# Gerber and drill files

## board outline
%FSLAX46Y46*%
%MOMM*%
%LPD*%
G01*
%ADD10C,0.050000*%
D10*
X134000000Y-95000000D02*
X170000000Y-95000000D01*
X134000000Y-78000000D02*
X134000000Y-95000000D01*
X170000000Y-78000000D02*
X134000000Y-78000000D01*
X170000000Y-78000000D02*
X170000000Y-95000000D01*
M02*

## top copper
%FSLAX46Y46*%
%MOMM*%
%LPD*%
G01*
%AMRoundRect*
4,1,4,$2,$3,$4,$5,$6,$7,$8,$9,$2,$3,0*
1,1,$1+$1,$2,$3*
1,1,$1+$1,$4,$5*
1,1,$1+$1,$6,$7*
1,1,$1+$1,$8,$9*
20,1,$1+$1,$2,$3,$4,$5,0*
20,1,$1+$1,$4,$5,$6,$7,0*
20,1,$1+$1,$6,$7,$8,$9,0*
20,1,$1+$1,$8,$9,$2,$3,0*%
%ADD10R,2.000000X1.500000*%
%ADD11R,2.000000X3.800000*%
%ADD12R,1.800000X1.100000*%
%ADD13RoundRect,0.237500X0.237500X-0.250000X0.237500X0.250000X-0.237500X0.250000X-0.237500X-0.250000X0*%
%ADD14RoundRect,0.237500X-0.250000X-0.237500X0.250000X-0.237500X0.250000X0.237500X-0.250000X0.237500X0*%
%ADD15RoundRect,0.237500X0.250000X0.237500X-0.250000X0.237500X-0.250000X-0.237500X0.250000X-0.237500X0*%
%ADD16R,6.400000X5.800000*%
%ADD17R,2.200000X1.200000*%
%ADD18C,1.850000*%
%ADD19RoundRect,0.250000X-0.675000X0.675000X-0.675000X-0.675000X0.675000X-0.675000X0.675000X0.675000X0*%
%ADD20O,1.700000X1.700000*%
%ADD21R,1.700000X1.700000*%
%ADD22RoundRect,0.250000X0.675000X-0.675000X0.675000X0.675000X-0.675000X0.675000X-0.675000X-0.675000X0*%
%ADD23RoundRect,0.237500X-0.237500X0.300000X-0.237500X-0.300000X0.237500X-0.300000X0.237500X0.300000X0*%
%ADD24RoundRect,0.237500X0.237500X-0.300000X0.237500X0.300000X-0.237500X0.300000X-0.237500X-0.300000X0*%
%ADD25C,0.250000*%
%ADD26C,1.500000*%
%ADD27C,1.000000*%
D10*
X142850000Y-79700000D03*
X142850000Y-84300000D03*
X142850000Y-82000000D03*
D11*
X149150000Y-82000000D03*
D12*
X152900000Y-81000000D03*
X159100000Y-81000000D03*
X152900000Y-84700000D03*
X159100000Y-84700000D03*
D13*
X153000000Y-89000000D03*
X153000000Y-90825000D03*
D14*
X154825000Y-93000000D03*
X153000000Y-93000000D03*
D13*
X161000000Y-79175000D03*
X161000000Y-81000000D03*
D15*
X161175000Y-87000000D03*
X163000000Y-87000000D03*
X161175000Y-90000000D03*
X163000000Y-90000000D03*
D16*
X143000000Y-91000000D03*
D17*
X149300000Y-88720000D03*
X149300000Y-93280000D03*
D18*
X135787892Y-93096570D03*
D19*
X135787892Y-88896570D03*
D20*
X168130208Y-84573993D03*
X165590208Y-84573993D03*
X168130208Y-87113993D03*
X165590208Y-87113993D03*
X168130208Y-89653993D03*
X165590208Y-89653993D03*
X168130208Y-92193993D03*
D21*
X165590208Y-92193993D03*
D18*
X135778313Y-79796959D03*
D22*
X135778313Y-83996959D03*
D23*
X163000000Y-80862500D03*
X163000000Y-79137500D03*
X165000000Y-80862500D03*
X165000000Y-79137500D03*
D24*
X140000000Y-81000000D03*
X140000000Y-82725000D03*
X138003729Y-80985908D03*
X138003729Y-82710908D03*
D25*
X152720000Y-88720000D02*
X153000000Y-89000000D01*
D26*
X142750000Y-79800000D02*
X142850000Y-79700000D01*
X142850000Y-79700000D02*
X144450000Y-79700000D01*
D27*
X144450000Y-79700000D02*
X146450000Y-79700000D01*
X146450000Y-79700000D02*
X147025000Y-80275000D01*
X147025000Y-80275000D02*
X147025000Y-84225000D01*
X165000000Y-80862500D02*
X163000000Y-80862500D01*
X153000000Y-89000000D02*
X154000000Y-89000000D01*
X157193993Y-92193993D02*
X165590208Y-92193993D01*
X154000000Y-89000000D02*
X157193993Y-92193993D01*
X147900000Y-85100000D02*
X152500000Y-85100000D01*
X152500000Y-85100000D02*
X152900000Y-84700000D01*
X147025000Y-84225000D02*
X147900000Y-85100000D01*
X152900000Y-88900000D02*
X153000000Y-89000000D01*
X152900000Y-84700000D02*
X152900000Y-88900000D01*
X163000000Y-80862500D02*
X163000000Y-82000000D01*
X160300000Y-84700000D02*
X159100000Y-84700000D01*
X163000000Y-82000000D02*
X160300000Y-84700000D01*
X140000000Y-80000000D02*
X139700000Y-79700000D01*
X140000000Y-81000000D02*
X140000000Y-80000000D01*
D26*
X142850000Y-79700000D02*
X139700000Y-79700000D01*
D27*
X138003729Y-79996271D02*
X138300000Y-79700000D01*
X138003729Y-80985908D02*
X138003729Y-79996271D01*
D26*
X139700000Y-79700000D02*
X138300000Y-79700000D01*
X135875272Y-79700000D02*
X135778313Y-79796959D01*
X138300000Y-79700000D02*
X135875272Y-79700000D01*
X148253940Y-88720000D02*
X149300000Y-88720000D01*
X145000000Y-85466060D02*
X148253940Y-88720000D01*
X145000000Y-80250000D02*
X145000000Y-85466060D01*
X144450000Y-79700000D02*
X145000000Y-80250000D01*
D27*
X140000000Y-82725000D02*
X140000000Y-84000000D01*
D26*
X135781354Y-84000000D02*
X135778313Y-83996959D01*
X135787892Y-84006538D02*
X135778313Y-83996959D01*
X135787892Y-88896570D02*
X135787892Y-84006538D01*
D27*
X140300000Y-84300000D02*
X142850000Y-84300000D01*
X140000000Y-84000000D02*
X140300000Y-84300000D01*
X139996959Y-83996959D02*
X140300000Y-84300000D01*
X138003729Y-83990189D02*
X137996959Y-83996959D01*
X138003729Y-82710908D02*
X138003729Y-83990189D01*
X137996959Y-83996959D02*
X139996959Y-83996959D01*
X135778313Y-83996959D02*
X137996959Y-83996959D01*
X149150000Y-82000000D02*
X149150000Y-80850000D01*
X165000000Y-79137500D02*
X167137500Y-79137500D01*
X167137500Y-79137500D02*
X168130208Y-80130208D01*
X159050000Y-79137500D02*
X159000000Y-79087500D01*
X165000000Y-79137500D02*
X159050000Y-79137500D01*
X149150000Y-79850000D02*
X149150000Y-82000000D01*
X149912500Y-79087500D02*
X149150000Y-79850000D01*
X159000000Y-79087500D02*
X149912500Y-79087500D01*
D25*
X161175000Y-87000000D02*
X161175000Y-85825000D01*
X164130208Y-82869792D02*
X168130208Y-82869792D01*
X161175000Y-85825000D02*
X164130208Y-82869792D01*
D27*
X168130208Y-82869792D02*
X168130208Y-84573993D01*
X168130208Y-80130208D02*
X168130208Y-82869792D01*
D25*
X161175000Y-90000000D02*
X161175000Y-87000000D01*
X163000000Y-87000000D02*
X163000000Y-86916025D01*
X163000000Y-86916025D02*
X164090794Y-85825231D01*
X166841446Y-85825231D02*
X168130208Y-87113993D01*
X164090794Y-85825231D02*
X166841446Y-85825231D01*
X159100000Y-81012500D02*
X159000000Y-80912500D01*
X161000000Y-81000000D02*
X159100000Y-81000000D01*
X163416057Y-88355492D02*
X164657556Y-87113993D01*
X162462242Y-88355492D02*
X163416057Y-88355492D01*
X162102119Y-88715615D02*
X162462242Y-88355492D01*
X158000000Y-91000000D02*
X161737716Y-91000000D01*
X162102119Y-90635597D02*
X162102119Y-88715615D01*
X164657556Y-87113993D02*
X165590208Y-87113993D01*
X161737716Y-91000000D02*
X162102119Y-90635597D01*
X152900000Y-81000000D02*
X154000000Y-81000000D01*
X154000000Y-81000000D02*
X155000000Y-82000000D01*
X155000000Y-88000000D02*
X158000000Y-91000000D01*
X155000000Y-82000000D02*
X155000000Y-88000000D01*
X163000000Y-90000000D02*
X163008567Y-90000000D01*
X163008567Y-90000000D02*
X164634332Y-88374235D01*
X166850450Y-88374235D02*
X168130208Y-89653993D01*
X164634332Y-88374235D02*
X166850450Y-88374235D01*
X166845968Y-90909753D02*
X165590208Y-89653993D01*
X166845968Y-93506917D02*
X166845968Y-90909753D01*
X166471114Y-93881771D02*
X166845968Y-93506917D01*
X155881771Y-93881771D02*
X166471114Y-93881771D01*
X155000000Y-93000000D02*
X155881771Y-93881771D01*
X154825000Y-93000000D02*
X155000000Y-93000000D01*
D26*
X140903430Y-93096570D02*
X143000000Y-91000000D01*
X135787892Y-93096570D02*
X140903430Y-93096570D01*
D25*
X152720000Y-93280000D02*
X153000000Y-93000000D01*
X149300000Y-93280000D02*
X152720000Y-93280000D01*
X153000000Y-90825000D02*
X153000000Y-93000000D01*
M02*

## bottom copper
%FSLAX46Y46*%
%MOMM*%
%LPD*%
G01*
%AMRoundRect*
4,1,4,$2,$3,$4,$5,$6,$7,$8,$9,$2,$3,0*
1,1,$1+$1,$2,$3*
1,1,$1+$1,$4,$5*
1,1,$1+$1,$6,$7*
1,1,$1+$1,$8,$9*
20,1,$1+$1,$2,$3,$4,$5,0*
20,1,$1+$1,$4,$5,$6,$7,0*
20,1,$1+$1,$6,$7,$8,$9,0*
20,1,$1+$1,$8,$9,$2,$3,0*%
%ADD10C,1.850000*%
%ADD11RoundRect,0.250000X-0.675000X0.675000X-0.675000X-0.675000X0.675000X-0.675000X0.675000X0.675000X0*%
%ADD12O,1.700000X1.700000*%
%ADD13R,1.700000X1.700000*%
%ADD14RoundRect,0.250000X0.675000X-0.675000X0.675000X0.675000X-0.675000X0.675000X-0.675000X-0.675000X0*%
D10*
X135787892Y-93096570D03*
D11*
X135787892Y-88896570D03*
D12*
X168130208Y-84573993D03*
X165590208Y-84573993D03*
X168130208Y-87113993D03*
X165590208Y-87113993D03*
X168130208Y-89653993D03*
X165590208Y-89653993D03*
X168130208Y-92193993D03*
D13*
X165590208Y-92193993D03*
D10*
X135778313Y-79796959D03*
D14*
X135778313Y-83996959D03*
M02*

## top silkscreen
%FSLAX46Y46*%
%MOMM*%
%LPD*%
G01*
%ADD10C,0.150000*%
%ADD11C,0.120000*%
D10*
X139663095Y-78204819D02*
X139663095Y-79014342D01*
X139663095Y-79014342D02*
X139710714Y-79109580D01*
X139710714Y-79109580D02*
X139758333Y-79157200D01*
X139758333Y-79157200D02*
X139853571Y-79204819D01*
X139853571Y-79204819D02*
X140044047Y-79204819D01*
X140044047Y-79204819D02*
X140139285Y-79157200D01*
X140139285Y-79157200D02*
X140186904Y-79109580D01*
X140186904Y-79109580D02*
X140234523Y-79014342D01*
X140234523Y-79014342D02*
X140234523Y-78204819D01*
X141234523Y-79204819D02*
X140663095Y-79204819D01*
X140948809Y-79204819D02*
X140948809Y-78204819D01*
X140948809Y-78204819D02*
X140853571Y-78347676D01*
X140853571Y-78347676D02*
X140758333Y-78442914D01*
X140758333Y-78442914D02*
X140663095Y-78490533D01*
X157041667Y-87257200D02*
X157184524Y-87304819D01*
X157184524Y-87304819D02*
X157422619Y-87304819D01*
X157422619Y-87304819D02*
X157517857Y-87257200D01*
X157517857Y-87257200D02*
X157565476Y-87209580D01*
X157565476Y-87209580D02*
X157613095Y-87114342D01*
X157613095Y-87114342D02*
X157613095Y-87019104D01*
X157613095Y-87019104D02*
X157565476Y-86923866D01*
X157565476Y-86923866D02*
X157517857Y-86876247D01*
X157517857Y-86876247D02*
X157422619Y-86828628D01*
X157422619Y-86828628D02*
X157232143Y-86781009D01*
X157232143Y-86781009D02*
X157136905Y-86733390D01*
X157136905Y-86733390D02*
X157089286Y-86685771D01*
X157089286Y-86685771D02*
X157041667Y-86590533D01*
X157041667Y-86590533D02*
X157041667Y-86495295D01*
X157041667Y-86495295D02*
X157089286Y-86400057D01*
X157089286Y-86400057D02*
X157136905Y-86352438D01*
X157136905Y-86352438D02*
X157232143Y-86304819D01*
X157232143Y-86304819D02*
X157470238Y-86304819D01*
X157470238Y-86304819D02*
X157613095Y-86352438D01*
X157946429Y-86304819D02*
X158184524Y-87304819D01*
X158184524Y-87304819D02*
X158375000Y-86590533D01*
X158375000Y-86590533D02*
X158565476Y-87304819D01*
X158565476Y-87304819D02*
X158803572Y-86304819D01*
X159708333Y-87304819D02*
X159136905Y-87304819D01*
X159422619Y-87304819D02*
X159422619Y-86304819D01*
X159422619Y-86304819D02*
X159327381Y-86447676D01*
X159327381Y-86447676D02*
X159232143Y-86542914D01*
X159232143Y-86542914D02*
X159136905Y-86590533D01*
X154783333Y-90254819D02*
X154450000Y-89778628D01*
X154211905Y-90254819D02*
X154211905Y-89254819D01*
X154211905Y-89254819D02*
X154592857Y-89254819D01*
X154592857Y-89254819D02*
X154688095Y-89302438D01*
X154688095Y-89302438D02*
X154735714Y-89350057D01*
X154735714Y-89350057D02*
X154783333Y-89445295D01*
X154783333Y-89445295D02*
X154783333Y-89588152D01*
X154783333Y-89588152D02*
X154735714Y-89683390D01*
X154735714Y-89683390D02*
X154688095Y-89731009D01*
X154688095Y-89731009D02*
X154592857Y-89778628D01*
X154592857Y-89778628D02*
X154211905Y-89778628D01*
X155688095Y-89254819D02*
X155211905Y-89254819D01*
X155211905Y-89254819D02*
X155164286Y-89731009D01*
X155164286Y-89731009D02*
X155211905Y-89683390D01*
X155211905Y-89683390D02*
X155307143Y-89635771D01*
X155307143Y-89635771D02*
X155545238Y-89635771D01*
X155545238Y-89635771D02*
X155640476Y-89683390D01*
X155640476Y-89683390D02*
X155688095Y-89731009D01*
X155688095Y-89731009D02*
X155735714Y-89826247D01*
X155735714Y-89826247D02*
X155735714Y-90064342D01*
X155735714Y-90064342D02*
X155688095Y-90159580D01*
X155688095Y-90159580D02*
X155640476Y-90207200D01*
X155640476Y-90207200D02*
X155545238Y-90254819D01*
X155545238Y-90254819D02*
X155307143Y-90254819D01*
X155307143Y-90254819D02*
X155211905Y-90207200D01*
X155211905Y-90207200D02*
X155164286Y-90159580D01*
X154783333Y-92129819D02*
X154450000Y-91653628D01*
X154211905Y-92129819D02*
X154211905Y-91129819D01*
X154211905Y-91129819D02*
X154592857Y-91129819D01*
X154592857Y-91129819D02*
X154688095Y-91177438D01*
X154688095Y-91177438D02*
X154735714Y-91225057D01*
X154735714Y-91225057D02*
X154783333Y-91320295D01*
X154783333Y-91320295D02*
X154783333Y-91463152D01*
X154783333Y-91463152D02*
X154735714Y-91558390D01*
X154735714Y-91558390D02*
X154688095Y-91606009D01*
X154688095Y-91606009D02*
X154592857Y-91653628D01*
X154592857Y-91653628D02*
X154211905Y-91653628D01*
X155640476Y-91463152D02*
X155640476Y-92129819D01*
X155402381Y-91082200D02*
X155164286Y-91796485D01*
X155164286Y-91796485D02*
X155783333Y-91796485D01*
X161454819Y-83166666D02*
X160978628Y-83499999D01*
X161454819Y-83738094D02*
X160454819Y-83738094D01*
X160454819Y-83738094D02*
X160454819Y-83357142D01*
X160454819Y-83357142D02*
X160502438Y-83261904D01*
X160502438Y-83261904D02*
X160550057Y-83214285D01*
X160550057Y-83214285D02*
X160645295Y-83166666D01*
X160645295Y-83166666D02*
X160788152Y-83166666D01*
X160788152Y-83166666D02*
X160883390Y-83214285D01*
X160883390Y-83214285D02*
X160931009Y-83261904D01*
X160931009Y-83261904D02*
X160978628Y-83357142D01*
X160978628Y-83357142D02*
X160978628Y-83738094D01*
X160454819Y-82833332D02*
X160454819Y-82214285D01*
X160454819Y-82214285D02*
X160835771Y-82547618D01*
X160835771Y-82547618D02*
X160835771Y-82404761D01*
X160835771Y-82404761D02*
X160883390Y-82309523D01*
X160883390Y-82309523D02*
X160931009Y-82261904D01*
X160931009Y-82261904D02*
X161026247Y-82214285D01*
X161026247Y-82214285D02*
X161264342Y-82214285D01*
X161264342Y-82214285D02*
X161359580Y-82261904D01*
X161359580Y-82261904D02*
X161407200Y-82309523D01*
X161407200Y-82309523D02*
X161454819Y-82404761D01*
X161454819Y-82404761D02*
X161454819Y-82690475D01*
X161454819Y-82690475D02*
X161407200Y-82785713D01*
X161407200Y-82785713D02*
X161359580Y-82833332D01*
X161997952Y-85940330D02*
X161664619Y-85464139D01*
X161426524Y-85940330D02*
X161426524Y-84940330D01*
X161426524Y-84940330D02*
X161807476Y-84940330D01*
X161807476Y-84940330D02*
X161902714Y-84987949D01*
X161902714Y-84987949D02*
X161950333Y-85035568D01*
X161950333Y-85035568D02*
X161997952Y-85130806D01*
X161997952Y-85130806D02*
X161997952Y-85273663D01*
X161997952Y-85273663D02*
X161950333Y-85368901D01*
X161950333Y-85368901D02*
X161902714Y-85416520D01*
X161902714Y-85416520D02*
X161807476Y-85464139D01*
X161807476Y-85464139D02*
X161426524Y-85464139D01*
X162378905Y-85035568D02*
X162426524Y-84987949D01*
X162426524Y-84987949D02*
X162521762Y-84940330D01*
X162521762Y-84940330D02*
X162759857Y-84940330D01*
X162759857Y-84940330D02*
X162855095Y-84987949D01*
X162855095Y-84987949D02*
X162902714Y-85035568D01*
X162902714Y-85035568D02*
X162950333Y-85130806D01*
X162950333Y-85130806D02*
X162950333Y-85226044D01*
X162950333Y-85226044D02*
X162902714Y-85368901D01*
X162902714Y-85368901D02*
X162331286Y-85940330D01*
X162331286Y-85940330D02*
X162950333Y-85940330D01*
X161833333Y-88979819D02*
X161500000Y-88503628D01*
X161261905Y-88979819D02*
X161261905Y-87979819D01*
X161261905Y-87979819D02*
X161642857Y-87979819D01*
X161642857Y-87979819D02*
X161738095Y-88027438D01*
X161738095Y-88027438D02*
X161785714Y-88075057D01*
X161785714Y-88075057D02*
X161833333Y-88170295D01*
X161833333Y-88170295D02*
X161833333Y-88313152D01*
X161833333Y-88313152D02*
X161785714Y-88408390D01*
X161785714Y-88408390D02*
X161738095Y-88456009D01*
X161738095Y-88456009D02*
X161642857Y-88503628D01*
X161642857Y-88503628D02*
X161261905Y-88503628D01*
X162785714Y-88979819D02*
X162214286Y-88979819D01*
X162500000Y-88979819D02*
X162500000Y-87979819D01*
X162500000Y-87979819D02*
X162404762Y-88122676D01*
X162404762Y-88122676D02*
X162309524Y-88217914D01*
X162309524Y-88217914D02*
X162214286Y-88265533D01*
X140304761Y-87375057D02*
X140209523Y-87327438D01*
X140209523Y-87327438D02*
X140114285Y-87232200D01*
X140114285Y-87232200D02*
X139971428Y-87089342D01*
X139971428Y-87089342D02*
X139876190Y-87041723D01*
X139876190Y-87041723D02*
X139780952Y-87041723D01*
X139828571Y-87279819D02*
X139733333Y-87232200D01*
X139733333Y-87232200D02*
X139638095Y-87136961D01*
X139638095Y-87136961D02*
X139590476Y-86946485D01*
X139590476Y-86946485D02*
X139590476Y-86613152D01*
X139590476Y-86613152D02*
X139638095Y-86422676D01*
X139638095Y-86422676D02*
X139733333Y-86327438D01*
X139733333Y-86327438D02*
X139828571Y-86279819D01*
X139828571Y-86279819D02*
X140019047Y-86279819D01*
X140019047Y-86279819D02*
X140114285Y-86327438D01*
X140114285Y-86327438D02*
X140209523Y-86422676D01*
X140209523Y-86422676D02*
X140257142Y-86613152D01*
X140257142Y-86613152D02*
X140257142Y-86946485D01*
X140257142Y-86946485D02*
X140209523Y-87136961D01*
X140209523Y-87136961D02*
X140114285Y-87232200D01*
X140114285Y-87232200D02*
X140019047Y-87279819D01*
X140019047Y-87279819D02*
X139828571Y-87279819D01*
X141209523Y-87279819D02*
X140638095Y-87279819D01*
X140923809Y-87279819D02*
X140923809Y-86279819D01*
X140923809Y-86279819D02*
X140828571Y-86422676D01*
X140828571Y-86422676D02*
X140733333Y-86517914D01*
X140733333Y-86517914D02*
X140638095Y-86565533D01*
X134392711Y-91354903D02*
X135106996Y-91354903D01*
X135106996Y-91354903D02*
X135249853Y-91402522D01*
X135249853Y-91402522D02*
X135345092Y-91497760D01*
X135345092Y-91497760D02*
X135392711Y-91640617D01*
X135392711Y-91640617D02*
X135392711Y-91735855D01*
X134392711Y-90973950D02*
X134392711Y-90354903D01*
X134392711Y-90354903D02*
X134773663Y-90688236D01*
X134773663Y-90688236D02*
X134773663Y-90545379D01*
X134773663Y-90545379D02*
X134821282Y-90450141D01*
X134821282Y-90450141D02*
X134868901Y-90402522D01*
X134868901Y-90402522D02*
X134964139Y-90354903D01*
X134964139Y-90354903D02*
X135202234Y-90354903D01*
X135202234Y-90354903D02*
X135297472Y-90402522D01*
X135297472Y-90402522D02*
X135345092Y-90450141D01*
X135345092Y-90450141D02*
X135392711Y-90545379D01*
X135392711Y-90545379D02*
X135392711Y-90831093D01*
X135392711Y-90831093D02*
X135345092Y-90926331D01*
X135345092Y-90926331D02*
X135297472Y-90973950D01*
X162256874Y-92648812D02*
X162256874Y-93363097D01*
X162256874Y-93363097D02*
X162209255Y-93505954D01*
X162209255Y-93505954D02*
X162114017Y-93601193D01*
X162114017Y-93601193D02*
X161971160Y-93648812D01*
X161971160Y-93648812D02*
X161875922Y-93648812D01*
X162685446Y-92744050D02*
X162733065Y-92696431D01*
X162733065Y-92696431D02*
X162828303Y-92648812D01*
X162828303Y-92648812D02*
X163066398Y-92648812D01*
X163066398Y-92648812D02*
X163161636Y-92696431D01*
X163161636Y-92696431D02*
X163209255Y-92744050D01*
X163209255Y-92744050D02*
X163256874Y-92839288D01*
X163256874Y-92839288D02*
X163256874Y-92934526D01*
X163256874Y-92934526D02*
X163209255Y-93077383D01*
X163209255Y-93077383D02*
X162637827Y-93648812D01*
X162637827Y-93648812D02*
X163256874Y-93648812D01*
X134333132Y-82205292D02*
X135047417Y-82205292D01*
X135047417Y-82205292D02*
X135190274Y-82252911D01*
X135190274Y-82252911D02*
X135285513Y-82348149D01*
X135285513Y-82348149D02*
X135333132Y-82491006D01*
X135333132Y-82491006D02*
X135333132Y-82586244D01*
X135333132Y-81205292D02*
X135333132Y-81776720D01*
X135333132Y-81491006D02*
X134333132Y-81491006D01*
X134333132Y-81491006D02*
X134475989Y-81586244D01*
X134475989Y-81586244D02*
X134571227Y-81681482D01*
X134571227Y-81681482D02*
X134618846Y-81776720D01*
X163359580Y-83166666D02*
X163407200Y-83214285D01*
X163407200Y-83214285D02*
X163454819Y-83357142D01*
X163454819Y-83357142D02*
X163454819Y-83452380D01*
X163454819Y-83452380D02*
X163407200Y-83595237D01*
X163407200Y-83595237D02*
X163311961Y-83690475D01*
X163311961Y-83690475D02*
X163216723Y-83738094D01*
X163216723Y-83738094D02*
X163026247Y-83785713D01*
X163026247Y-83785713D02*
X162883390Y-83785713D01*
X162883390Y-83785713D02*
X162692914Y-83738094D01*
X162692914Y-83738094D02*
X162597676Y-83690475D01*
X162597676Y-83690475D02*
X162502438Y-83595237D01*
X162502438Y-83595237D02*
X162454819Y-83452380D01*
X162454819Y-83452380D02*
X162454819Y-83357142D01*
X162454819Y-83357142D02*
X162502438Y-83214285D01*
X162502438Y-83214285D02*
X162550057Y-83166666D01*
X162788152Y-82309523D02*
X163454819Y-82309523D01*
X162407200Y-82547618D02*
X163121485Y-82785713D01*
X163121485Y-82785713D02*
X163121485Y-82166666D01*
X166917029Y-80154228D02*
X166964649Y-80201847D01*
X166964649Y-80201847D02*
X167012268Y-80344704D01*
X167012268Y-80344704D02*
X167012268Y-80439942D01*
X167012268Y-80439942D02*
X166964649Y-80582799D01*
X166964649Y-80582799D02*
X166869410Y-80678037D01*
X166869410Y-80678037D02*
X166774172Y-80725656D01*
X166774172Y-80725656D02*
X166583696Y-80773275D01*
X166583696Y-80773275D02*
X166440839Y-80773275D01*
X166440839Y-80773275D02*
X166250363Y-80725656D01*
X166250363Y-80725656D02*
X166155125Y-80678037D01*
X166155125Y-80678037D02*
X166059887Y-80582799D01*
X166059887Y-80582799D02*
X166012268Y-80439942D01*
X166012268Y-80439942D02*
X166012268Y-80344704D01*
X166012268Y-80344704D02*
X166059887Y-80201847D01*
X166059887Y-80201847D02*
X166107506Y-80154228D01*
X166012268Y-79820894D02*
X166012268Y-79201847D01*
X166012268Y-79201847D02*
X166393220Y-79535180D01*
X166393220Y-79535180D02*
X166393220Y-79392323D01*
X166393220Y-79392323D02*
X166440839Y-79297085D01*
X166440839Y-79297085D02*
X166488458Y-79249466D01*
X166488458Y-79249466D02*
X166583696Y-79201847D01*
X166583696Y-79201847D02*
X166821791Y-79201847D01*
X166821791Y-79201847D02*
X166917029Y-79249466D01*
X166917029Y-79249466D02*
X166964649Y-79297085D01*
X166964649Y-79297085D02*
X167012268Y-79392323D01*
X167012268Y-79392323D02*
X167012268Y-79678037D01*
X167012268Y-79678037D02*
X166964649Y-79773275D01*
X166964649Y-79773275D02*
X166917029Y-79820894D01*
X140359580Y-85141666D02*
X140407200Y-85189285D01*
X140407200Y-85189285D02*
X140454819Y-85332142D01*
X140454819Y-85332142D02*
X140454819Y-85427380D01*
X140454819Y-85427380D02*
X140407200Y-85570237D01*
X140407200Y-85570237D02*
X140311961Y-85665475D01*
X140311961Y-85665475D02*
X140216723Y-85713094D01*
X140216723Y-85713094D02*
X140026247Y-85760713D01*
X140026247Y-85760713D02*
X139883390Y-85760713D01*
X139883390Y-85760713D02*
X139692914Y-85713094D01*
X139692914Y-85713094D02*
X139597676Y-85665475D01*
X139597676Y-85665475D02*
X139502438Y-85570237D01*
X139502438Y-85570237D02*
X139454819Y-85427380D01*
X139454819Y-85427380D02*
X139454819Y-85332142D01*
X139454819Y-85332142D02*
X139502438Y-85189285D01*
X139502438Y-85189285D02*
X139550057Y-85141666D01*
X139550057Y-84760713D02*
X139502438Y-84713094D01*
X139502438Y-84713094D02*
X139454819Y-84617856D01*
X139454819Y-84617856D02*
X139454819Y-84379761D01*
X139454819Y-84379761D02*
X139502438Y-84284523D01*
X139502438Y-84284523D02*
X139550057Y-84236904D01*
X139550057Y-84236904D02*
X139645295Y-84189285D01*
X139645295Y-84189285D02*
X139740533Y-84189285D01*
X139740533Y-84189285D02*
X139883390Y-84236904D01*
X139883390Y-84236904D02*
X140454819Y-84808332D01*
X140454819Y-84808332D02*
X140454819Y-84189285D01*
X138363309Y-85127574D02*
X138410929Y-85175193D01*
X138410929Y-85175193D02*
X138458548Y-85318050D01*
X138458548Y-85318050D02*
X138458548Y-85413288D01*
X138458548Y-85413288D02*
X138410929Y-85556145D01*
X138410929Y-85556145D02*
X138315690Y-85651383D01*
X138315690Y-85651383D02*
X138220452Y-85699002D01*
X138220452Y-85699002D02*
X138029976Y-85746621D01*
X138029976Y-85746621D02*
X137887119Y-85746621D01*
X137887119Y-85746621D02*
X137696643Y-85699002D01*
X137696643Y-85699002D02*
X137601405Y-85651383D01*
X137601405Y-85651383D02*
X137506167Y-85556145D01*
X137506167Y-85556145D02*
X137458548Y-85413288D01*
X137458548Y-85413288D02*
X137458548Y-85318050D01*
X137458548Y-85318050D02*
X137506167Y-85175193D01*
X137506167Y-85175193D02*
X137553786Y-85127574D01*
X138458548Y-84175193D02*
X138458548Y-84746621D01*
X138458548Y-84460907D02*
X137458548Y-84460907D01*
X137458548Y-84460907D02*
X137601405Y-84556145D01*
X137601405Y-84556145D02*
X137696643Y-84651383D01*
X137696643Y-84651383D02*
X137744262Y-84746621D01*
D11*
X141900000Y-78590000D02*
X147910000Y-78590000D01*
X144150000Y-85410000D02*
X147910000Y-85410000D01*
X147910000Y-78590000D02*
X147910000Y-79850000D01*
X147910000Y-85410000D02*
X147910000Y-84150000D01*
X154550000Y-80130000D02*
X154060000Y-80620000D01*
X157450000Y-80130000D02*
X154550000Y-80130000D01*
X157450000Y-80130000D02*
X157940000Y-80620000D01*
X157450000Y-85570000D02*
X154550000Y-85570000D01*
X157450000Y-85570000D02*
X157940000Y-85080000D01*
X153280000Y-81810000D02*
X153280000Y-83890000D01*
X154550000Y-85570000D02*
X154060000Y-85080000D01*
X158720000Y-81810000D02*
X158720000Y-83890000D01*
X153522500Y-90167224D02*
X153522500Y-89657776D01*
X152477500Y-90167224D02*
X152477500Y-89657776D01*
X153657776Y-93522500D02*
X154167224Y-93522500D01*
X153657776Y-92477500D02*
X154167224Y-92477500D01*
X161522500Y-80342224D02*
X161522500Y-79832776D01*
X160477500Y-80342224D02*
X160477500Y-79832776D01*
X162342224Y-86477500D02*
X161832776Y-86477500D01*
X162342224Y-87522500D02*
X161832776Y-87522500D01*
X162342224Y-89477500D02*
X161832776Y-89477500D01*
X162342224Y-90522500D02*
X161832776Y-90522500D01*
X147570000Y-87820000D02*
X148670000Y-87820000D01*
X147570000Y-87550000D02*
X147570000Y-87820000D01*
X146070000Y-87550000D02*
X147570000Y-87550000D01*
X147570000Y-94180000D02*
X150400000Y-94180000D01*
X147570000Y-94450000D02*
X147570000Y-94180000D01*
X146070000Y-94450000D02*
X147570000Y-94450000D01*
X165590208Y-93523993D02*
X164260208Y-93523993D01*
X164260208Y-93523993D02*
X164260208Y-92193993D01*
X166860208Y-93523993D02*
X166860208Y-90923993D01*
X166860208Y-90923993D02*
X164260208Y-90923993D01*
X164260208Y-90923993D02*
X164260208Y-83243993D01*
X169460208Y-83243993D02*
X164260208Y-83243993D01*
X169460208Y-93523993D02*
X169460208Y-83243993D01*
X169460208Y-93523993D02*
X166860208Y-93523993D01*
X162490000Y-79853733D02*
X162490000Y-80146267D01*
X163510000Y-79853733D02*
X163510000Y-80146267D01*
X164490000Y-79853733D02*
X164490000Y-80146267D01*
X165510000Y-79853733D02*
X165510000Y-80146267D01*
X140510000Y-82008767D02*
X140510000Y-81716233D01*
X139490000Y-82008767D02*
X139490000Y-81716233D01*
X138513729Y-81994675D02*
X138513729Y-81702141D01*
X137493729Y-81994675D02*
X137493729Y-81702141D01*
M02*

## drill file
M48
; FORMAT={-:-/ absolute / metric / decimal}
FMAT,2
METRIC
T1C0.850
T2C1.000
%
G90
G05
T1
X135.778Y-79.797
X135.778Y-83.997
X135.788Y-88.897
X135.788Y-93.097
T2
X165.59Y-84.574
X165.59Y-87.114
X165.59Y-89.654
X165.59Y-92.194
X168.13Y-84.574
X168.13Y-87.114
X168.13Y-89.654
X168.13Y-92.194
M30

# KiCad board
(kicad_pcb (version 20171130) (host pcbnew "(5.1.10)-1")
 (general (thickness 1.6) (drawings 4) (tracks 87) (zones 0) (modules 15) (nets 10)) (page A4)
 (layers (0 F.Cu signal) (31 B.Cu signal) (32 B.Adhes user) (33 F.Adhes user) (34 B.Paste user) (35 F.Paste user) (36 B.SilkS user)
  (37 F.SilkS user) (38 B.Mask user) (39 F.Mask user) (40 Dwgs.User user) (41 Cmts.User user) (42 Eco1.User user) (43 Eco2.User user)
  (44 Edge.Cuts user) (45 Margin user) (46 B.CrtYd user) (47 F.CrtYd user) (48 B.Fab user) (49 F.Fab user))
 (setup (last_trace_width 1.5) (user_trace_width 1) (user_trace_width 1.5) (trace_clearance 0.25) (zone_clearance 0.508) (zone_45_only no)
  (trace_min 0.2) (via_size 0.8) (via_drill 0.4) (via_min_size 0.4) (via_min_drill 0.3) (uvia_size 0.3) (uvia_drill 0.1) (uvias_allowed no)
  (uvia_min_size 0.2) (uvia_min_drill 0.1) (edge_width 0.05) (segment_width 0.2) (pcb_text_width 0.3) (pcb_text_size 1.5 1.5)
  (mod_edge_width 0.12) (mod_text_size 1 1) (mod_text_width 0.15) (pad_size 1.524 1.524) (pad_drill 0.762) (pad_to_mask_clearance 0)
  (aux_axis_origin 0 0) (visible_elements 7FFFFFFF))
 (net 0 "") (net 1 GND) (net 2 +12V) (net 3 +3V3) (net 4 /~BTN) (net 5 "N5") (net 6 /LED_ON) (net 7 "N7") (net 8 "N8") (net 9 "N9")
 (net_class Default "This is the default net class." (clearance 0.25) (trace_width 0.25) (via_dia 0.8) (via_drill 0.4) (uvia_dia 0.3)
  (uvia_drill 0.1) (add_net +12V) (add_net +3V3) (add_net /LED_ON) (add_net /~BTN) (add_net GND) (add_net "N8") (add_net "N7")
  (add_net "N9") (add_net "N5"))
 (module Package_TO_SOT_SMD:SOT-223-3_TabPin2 (layer F.Cu) (at 146 82)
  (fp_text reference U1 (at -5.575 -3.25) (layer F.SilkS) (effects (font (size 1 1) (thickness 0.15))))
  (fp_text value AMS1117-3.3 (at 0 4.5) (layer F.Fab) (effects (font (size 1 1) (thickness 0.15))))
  (fp_line (start -4.1 -3.41) (end 1.91 -3.41) (layer F.SilkS) (width 0.12))
  (fp_line (start -1.85 3.41) (end 1.91 3.41) (layer F.SilkS) (width 0.12))
  (fp_line (start 1.91 -3.41) (end 1.91 -2.15) (layer F.SilkS) (width 0.12))
  (fp_line (start 1.91 3.41) (end 1.91 2.15) (layer F.SilkS) (width 0.12))
  (pad 1 smd rect (at -3.15 -2.3) (size 2 1.5) (layers F.Cu F.Paste F.Mask) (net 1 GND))
  (pad 3 smd rect (at -3.15 2.3) (size 2 1.5) (layers F.Cu F.Paste F.Mask) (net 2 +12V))
  (pad 2 smd rect (at -3.15 0) (size 2 1.5) (layers F.Cu F.Paste F.Mask) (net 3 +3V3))
  (pad 2 smd rect (at 3.15 0) (size 2 3.8) (layers F.Cu F.Paste F.Mask) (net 3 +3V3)))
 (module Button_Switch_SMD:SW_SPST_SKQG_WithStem (layer F.Cu) (at 156 82.85 180)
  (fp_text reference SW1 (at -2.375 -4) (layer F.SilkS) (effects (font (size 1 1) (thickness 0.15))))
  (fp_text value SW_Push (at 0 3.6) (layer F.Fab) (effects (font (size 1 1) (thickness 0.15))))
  (fp_line (start 1.45 2.72) (end 1.94 2.23) (layer F.SilkS) (width 0.12))
  (fp_line (start -1.45 2.72) (end 1.45 2.72) (layer F.SilkS) (width 0.12))
  (fp_line (start -1.45 2.72) (end -1.94 2.23) (layer F.SilkS) (width 0.12))
  (fp_line (start -1.45 -2.72) (end 1.45 -2.72) (layer F.SilkS) (width 0.12))
  (fp_line (start -1.45 -2.72) (end -1.94 -2.23) (layer F.SilkS) (width 0.12))
  (fp_line (start 2.72 1.04) (end 2.72 -1.04) (layer F.SilkS) (width 0.12))
  (fp_line (start 1.45 -2.72) (end 1.94 -2.23) (layer F.SilkS) (width 0.12))
  (fp_line (start -2.72 1.04) (end -2.72 -1.04) (layer F.SilkS) (width 0.12))
  (pad 2 smd rect (at 3.1 1.85 180) (size 1.8 1.1) (layers F.Cu F.Paste F.Mask) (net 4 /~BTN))
  (pad 2 smd rect (at -3.1 1.85 180) (size 1.8 1.1) (layers F.Cu F.Paste F.Mask) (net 4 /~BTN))
  (pad 1 smd rect (at 3.1 -1.85 180) (size 1.8 1.1) (layers F.Cu F.Paste F.Mask) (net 1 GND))
  (pad 1 smd rect (at -3.1 -1.85 180) (size 1.8 1.1) (layers F.Cu F.Paste F.Mask) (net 1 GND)))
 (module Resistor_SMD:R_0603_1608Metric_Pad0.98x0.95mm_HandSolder (layer F.Cu) (at 153 89.9125 90)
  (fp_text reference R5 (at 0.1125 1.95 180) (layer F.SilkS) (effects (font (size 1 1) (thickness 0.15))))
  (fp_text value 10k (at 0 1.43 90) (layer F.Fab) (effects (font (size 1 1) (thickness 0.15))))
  (fp_line (start -0.254724 0.5225) (end 0.254724 0.5225) (layer F.SilkS) (width 0.12))
  (fp_line (start -0.254724 -0.5225) (end 0.254724 -0.5225) (layer F.SilkS) (width 0.12))
  (pad 2 smd roundrect (at 0.9125 0 90) (size 0.975 0.95) (layers F.Cu F.Paste F.Mask) (roundrect_rratio 0.25) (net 1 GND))
  (pad 1 smd roundrect (at -0.9125 0 90) (size 0.975 0.95) (layers F.Cu F.Paste F.Mask) (roundrect_rratio 0.25) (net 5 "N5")))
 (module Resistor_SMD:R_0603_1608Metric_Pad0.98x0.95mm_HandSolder (layer F.Cu) (at 153.9125 93)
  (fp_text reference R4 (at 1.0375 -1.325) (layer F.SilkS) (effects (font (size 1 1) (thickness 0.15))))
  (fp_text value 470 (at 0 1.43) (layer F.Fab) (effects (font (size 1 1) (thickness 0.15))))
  (fp_line (start -0.254724 0.5225) (end 0.254724 0.5225) (layer F.SilkS) (width 0.12))
  (fp_line (start -0.254724 -0.5225) (end 0.254724 -0.5225) (layer F.SilkS) (width 0.12))
  (pad 2 smd roundrect (at 0.9125 0) (size 0.975 0.95) (layers F.Cu F.Paste F.Mask) (roundrect_rratio 0.25) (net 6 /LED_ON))
  (pad 1 smd roundrect (at -0.9125 0) (size 0.975 0.95) (layers F.Cu F.Paste F.Mask) (roundrect_rratio 0.25) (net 5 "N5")))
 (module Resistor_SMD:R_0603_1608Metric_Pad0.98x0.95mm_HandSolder (layer F.Cu) (at 161 80.0875 90)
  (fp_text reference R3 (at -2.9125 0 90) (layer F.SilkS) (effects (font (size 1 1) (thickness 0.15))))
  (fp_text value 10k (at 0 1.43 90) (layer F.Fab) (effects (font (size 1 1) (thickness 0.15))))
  (fp_line (start -0.254724 0.5225) (end 0.254724 0.5225) (layer F.SilkS) (width 0.12))
  (fp_line (start -0.254724 -0.5225) (end 0.254724 -0.5225) (layer F.SilkS) (width 0.12))
  (pad 2 smd roundrect (at 0.9125 0 90) (size 0.975 0.95) (layers F.Cu F.Paste F.Mask) (roundrect_rratio 0.25) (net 3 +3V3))
  (pad 1 smd roundrect (at -0.9125 0 90) (size 0.975 0.95) (layers F.Cu F.Paste F.Mask) (roundrect_rratio 0.25) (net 4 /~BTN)))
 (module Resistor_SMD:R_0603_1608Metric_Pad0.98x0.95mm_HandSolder (layer F.Cu) (at 162.0875 87 180)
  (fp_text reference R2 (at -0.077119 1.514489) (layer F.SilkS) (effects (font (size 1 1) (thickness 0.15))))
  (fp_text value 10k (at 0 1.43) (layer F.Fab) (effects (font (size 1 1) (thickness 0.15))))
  (fp_line (start -0.254724 0.5225) (end 0.254724 0.5225) (layer F.SilkS) (width 0.12))
  (fp_line (start -0.254724 -0.5225) (end 0.254724 -0.5225) (layer F.SilkS) (width 0.12))
  (pad 2 smd roundrect (at 0.9125 0 180) (size 0.975 0.95) (layers F.Cu F.Paste F.Mask) (roundrect_rratio 0.25) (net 3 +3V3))
  (pad 1 smd roundrect (at -0.9125 0 180) (size 0.975 0.95) (layers F.Cu F.Paste F.Mask) (roundrect_rratio 0.25) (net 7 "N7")))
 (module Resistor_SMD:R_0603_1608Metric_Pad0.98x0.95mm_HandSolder (layer F.Cu) (at 162.0875 90 180)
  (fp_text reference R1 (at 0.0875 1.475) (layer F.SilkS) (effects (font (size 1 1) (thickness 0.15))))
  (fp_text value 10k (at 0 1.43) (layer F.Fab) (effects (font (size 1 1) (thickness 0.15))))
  (fp_line (start -0.254724 0.5225) (end 0.254724 0.5225) (layer F.SilkS) (width 0.12))
  (fp_line (start -0.254724 -0.5225) (end 0.254724 -0.5225) (layer F.SilkS) (width 0.12))
  (pad 2 smd roundrect (at 0.9125 0 180) (size 0.975 0.95) (layers F.Cu F.Paste F.Mask) (roundrect_rratio 0.25) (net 3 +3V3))
  (pad 1 smd roundrect (at -0.9125 0 180) (size 0.975 0.95) (layers F.Cu F.Paste F.Mask) (roundrect_rratio 0.25) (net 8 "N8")))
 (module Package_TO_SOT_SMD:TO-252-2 (layer F.Cu) (at 145.1 91 180)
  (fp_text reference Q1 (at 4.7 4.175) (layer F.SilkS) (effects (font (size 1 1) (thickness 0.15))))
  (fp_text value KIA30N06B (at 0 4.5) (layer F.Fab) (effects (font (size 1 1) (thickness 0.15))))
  (fp_line (start -2.47 3.18) (end -3.57 3.18) (layer F.SilkS) (width 0.12))
  (fp_line (start -2.47 3.45) (end -2.47 3.18) (layer F.SilkS) (width 0.12))
  (fp_line (start -0.97 3.45) (end -2.47 3.45) (layer F.SilkS) (width 0.12))
  (fp_line (start -2.47 -3.18) (end -5.3 -3.18) (layer F.SilkS) (width 0.12))
  (fp_line (start -2.47 -3.45) (end -2.47 -3.18) (layer F.SilkS) (width 0.12))
  (fp_line (start -0.97 -3.45) (end -2.47 -3.45) (layer F.SilkS) (width 0.12))
  (pad "" smd rect (at 0.425 1.525 180) (size 3.05 2.75) (layers F.Paste))
  (pad "" smd rect (at 3.775 -1.525 180) (size 3.05 2.75) (layers F.Paste))
  (pad "" smd rect (at 0.425 -1.525 180) (size 3.05 2.75) (layers F.Paste))
  (pad "" smd rect (at 3.775 1.525 180) (size 3.05 2.75) (layers F.Paste))
  (pad 2 smd rect (at 2.1 0 180) (size 6.4 5.8) (layers F.Cu F.Mask) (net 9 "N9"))
  (pad 3 smd rect (at -4.2 2.28 180) (size 2.2 1.2) (layers F.Cu F.Paste F.Mask) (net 1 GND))
  (pad 1 smd rect (at -4.2 -2.28 180) (size 2.2 1.2) (layers F.Cu F.Paste F.Mask) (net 5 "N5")))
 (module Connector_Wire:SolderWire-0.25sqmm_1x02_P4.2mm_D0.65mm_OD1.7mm (layer F.Cu) (at 135.787892 88.89657 270)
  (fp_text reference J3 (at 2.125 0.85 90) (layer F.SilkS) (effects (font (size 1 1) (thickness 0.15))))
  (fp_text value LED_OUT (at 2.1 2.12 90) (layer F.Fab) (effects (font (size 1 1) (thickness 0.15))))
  (pad 2 thru_hole circle (at 4.2 0 270) (size 1.85 1.85) (drill 0.85) (layers *.Cu *.Mask) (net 9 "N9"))
  (pad 1 thru_hole roundrect (at 0 0 270) (size 1.85 1.85) (drill 0.85) (layers *.Cu *.Mask) (roundrect_rratio 0.135135) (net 2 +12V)))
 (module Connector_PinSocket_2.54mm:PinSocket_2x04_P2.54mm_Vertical (layer F.Cu) (at 165.590208 92.193993 180)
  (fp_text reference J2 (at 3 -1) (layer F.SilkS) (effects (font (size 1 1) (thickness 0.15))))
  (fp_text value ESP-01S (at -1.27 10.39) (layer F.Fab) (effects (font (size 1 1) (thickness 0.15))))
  (fp_line (start 0 -1.33) (end 1.33 -1.33) (layer F.SilkS) (width 0.12))
  (fp_line (start 1.33 -1.33) (end 1.33 0) (layer F.SilkS) (width 0.12))
  (fp_line (start -1.27 -1.33) (end -1.27 1.27) (layer F.SilkS) (width 0.12))
  (fp_line (start -1.27 1.27) (end 1.33 1.27) (layer F.SilkS) (width 0.12))
  (fp_line (start 1.33 1.27) (end 1.33 8.95) (layer F.SilkS) (width 0.12))
  (fp_line (start -3.87 8.95) (end 1.33 8.95) (layer F.SilkS) (width 0.12))
  (fp_line (start -3.87 -1.33) (end -3.87 8.95) (layer F.SilkS) (width 0.12))
  (fp_line (start -3.87 -1.33) (end -1.27 -1.33) (layer F.SilkS) (width 0.12))
  (pad 8 thru_hole oval (at -2.54 7.62 180) (size 1.7 1.7) (drill 1) (layers *.Cu *.Mask) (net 3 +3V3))
  (pad 7 thru_hole oval (at 0 7.62 180) (size 1.7 1.7) (drill 1) (layers *.Cu *.Mask))
  (pad 6 thru_hole oval (at -2.54 5.08 180) (size 1.7 1.7) (drill 1) (layers *.Cu *.Mask) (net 7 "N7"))
  (pad 5 thru_hole oval (at 0 5.08 180) (size 1.7 1.7) (drill 1) (layers *.Cu *.Mask) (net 4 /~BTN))
  (pad 4 thru_hole oval (at -2.54 2.54 180) (size 1.7 1.7) (drill 1) (layers *.Cu *.Mask) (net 8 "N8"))
  (pad 3 thru_hole oval (at 0 2.54 180) (size 1.7 1.7) (drill 1) (layers *.Cu *.Mask) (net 6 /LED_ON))
  (pad 2 thru_hole oval (at -2.54 0 180) (size 1.7 1.7) (drill 1) (layers *.Cu *.Mask))
  (pad 1 thru_hole rect (at 0 0 180) (size 1.7 1.7) (drill 1) (layers *.Cu *.Mask) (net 1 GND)))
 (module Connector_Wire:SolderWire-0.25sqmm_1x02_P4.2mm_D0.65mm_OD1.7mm (layer F.Cu) (at 135.778313 83.996959 90)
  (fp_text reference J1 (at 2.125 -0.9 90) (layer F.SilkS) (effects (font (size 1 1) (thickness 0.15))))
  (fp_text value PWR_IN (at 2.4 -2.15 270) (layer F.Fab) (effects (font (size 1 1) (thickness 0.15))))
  (pad 2 thru_hole circle (at 4.2 0 90) (size 1.85 1.85) (drill 0.85) (layers *.Cu *.Mask) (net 1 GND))
  (pad 1 thru_hole roundrect (at 0 0 90) (size 1.85 1.85) (drill 0.85) (layers *.Cu *.Mask) (roundrect_rratio 0.135135) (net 2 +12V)))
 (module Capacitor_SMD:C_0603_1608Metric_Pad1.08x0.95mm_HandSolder (layer F.Cu) (at 163 80 270)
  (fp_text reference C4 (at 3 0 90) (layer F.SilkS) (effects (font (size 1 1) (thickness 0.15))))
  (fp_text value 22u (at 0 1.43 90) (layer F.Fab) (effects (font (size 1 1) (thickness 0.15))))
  (fp_line (start -0.146267 0.51) (end 0.146267 0.51) (layer F.SilkS) (width 0.12))
  (fp_line (start -0.146267 -0.51) (end 0.146267 -0.51) (layer F.SilkS) (width 0.12))
  (pad 2 smd roundrect (at 0.8625 0 270) (size 1.075 0.95) (layers F.Cu F.Paste F.Mask) (roundrect_rratio 0.25) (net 1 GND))
  (pad 1 smd roundrect (at -0.8625 0 270) (size 1.075 0.95) (layers F.Cu F.Paste F.Mask) (roundrect_rratio 0.25) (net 3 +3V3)))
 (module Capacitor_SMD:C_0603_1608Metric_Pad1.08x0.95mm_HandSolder (layer F.Cu) (at 165 80 270)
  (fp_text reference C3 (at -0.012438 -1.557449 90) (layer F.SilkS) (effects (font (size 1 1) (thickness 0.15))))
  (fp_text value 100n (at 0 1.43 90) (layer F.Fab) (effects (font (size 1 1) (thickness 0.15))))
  (fp_line (start -0.146267 0.51) (end 0.146267 0.51) (layer F.SilkS) (width 0.12))
  (fp_line (start -0.146267 -0.51) (end 0.146267 -0.51) (layer F.SilkS) (width 0.12))
  (pad 2 smd roundrect (at 0.8625 0 270) (size 1.075 0.95) (layers F.Cu F.Paste F.Mask) (roundrect_rratio 0.25) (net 1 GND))
  (pad 1 smd roundrect (at -0.8625 0 270) (size 1.075 0.95) (layers F.Cu F.Paste F.Mask) (roundrect_rratio 0.25) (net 3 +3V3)))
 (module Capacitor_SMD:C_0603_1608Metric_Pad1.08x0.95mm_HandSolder (layer F.Cu) (at 140 81.8625 90)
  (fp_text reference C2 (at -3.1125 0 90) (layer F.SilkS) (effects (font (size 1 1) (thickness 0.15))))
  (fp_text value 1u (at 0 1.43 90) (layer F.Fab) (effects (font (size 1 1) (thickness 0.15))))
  (fp_line (start -0.146267 0.51) (end 0.146267 0.51) (layer F.SilkS) (width 0.12))
  (fp_line (start -0.146267 -0.51) (end 0.146267 -0.51) (layer F.SilkS) (width 0.12))
  (pad 2 smd roundrect (at 0.8625 0 90) (size 1.075 0.95) (layers F.Cu F.Paste F.Mask) (roundrect_rratio 0.25) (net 1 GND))
  (pad 1 smd roundrect (at -0.8625 0 90) (size 1.075 0.95) (layers F.Cu F.Paste F.Mask) (roundrect_rratio 0.25) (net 2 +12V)))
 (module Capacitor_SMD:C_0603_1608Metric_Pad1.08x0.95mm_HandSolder (layer F.Cu) (at 138.003729 81.848408 90)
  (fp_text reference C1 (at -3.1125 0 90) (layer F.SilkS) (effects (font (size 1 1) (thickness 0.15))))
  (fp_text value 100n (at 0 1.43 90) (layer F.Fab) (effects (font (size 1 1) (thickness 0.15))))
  (fp_line (start -0.146267 0.51) (end 0.146267 0.51) (layer F.SilkS) (width 0.12))
  (fp_line (start -0.146267 -0.51) (end 0.146267 -0.51) (layer F.SilkS) (width 0.12))
  (pad 2 smd roundrect (at 0.8625 0 90) (size 1.075 0.95) (layers F.Cu F.Paste F.Mask) (roundrect_rratio 0.25) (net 1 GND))
  (pad 1 smd roundrect (at -0.8625 0 90) (size 1.075 0.95) (layers F.Cu F.Paste F.Mask) (roundrect_rratio 0.25) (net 2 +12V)))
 (gr_line (start 134 95) (end 170 95) (layer Edge.Cuts) (width 0.05))
 (gr_line (start 134 78) (end 134 95) (layer Edge.Cuts) (width 0.05))
 (gr_line (start 170 78) (end 134 78) (layer Edge.Cuts) (width 0.05))
 (gr_line (start 170 78) (end 170 95) (layer Edge.Cuts) (width 0.05))
 (segment (start 152.72 88.72) (end 153 89) (width 0.25) (layer F.Cu) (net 1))
 (segment (start 142.75 79.8) (end 142.85 79.7) (width 1.5) (layer F.Cu) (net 1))
 (segment (start 142.85 79.7) (end 144.45 79.7) (width 1.5) (layer F.Cu) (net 1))
 (segment (start 144.45 79.7) (end 146.45 79.7) (width 1) (layer F.Cu) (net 1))
 (segment (start 146.45 79.7) (end 147.025 80.275) (width 1) (layer F.Cu) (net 1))
 (segment (start 147.025 80.275) (end 147.025 84.225) (width 1) (layer F.Cu) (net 1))
 (segment (start 165 80.8625) (end 163 80.8625) (width 1) (layer F.Cu) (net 1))
 (segment (start 153 89) (end 154 89) (width 1) (layer F.Cu) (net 1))
 (segment (start 157.193993 92.193993) (end 165.590208 92.193993) (width 1) (layer F.Cu) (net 1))
 (segment (start 154 89) (end 157.193993 92.193993) (width 1) (layer F.Cu) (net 1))
 (segment (start 147.9 85.1) (end 152.5 85.1) (width 1) (layer F.Cu) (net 1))
 (segment (start 152.5 85.1) (end 152.9 84.7) (width 1) (layer F.Cu) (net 1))
 (segment (start 147.025 84.225) (end 147.9 85.1) (width 1) (layer F.Cu) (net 1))
 (segment (start 152.9 88.9) (end 153 89) (width 1) (layer F.Cu) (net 1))
 (segment (start 152.9 84.7) (end 152.9 88.9) (width 1) (layer F.Cu) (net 1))
 (segment (start 163 80.8625) (end 163 82) (width 1) (layer F.Cu) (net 1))
 (segment (start 160.3 84.7) (end 159.1 84.7) (width 1) (layer F.Cu) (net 1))
 (segment (start 163 82) (end 160.3 84.7) (width 1) (layer F.Cu) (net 1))
 (segment (start 140 80) (end 139.7 79.7) (width 1) (layer F.Cu) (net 1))
 (segment (start 140 81) (end 140 80) (width 1) (layer F.Cu) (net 1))
 (segment (start 142.85 79.7) (end 139.7 79.7) (width 1.5) (layer F.Cu) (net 1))
 (segment (start 138.003729 79.996271) (end 138.3 79.7) (width 1) (layer F.Cu) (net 1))
 (segment (start 138.003729 80.985908) (end 138.003729 79.996271) (width 1) (layer F.Cu) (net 1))
 (segment (start 139.7 79.7) (end 138.3 79.7) (width 1.5) (layer F.Cu) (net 1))
 (segment (start 135.875272 79.7) (end 135.778313 79.796959) (width 1.5) (layer F.Cu) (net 1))
 (segment (start 138.3 79.7) (end 135.875272 79.7) (width 1.5) (layer F.Cu) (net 1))
 (segment (start 148.25394 88.72) (end 149.3 88.72) (width 1.5) (layer F.Cu) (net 1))
 (segment (start 145 85.46606) (end 148.25394 88.72) (width 1.5) (layer F.Cu) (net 1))
 (segment (start 145 80.25) (end 145 85.46606) (width 1.5) (layer F.Cu) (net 1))
 (segment (start 144.45 79.7) (end 145 80.25) (width 1.5) (layer F.Cu) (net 1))
 (segment (start 140 82.725) (end 140 84) (width 1) (layer F.Cu) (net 2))
 (segment (start 135.781354 84) (end 135.778313 83.996959) (width 1.5) (layer F.Cu) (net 2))
 (segment (start 135.787892 84.006538) (end 135.778313 83.996959) (width 1.5) (layer F.Cu) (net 2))
 (segment (start 135.787892 88.89657) (end 135.787892 84.006538) (width 1.5) (layer F.Cu) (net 2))
 (segment (start 140.3 84.3) (end 142.85 84.3) (width 1) (layer F.Cu) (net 2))
 (segment (start 140 84) (end 140.3 84.3) (width 1) (layer F.Cu) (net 2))
 (segment (start 139.996959 83.996959) (end 140.3 84.3) (width 1) (layer F.Cu) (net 2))
 (segment (start 138.003729 83.990189) (end 137.996959 83.996959) (width 1) (layer F.Cu) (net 2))
 (segment (start 138.003729 82.710908) (end 138.003729 83.990189) (width 1) (layer F.Cu) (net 2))
 (segment (start 137.996959 83.996959) (end 139.996959 83.996959) (width 1) (layer F.Cu) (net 2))
 (segment (start 135.778313 83.996959) (end 137.996959 83.996959) (width 1) (layer F.Cu) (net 2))
 (segment (start 149.15 82) (end 149.15 80.85) (width 1) (layer F.Cu) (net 3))
 (segment (start 165 79.1375) (end 167.1375 79.1375) (width 1) (layer F.Cu) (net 3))
 (segment (start 167.1375 79.1375) (end 168.130208 80.130208) (width 1) (layer F.Cu) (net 3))
 (segment (start 159.05 79.1375) (end 159 79.0875) (width 1) (layer F.Cu) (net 3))
 (segment (start 165 79.1375) (end 159.05 79.1375) (width 1) (layer F.Cu) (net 3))
 (segment (start 149.15 79.85) (end 149.15 82) (width 1) (layer F.Cu) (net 3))
 (segment (start 149.9125 79.0875) (end 149.15 79.85) (width 1) (layer F.Cu) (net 3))
 (segment (start 159 79.0875) (end 149.9125 79.0875) (width 1) (layer F.Cu) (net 3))
 (segment (start 161.175 87) (end 161.175 85.825) (width 0.25) (layer F.Cu) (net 3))
 (segment (start 164.130208 82.869792) (end 168.130208 82.869792) (width 0.25) (layer F.Cu) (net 3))
 (segment (start 161.175 85.825) (end 164.130208 82.869792) (width 0.25) (layer F.Cu) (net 3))
 (segment (start 168.130208 82.869792) (end 168.130208 84.573993) (width 1) (layer F.Cu) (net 3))
 (segment (start 168.130208 80.130208) (end 168.130208 82.869792) (width 1) (layer F.Cu) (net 3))
 (segment (start 161.175 90) (end 161.175 87) (width 0.25) (layer F.Cu) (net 3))
 (segment (start 163 87) (end 163 86.916025) (width 0.25) (layer F.Cu) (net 7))
 (segment (start 163 86.916025) (end 164.090794 85.825231) (width 0.25) (layer F.Cu) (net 7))
 (segment (start 166.841446 85.825231) (end 168.130208 87.113993) (width 0.25) (layer F.Cu) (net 7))
 (segment (start 164.090794 85.825231) (end 166.841446 85.825231) (width 0.25) (layer F.Cu) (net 7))
 (segment (start 159.1 81.0125) (end 159 80.9125) (width 0.25) (layer F.Cu) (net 4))
 (segment (start 161 81) (end 159.1 81) (width 0.25) (layer F.Cu) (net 4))
 (segment (start 163.416057 88.355492) (end 164.657556 87.113993) (width 0.25) (layer F.Cu) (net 4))
 (segment (start 162.462242 88.355492) (end 163.416057 88.355492) (width 0.25) (layer F.Cu) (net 4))
 (segment (start 162.102119 88.715615) (end 162.462242 88.355492) (width 0.25) (layer F.Cu) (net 4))
 (segment (start 158 91) (end 161.737716 91) (width 0.25) (layer F.Cu) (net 4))
 (segment (start 162.102119 90.635597) (end 162.102119 88.715615) (width 0.25) (layer F.Cu) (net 4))
 (segment (start 164.657556 87.113993) (end 165.590208 87.113993) (width 0.25) (layer F.Cu) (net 4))
 (segment (start 161.737716 91) (end 162.102119 90.635597) (width 0.25) (layer F.Cu) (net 4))
 (segment (start 152.9 81) (end 154 81) (width 0.25) (layer F.Cu) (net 4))
 (segment (start 154 81) (end 155 82) (width 0.25) (layer F.Cu) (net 4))
 (segment (start 155 88) (end 158 91) (width 0.25) (layer F.Cu) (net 4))
 (segment (start 155 82) (end 155 88) (width 0.25) (layer F.Cu) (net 4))
 (segment (start 163 90) (end 163.008567 90) (width 0.25) (layer F.Cu) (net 8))
 (segment (start 163.008567 90) (end 164.634332 88.374235) (width 0.25) (layer F.Cu) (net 8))
 (segment (start 166.85045 88.374235) (end 168.130208 89.653993) (width 0.25) (layer F.Cu) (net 8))
 (segment (start 164.634332 88.374235) (end 166.85045 88.374235) (width 0.25) (layer F.Cu) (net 8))
 (segment (start 166.845968 90.909753) (end 165.590208 89.653993) (width 0.25) (layer F.Cu) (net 6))
 (segment (start 166.845968 93.506917) (end 166.845968 90.909753) (width 0.25) (layer F.Cu) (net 6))
 (segment (start 166.471114 93.881771) (end 166.845968 93.506917) (width 0.25) (layer F.Cu) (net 6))
 (segment (start 155.881771 93.881771) (end 166.471114 93.881771) (width 0.25) (layer F.Cu) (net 6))
 (segment (start 155 93) (end 155.881771 93.881771) (width 0.25) (layer F.Cu) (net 6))
 (segment (start 154.825 93) (end 155 93) (width 0.25) (layer F.Cu) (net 6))
 (segment (start 140.90343 93.09657) (end 143 91) (width 1.5) (layer F.Cu) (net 9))
 (segment (start 135.787892 93.09657) (end 140.90343 93.09657) (width 1.5) (layer F.Cu) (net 9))
 (segment (start 152.72 93.28) (end 153 93) (width 0.25) (layer F.Cu) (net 5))
 (segment (start 149.3 93.28) (end 152.72 93.28) (width 0.25) (layer F.Cu) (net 5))
 (segment (start 153 90.825) (end 153 93) (width 0.25) (layer F.Cu) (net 5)))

